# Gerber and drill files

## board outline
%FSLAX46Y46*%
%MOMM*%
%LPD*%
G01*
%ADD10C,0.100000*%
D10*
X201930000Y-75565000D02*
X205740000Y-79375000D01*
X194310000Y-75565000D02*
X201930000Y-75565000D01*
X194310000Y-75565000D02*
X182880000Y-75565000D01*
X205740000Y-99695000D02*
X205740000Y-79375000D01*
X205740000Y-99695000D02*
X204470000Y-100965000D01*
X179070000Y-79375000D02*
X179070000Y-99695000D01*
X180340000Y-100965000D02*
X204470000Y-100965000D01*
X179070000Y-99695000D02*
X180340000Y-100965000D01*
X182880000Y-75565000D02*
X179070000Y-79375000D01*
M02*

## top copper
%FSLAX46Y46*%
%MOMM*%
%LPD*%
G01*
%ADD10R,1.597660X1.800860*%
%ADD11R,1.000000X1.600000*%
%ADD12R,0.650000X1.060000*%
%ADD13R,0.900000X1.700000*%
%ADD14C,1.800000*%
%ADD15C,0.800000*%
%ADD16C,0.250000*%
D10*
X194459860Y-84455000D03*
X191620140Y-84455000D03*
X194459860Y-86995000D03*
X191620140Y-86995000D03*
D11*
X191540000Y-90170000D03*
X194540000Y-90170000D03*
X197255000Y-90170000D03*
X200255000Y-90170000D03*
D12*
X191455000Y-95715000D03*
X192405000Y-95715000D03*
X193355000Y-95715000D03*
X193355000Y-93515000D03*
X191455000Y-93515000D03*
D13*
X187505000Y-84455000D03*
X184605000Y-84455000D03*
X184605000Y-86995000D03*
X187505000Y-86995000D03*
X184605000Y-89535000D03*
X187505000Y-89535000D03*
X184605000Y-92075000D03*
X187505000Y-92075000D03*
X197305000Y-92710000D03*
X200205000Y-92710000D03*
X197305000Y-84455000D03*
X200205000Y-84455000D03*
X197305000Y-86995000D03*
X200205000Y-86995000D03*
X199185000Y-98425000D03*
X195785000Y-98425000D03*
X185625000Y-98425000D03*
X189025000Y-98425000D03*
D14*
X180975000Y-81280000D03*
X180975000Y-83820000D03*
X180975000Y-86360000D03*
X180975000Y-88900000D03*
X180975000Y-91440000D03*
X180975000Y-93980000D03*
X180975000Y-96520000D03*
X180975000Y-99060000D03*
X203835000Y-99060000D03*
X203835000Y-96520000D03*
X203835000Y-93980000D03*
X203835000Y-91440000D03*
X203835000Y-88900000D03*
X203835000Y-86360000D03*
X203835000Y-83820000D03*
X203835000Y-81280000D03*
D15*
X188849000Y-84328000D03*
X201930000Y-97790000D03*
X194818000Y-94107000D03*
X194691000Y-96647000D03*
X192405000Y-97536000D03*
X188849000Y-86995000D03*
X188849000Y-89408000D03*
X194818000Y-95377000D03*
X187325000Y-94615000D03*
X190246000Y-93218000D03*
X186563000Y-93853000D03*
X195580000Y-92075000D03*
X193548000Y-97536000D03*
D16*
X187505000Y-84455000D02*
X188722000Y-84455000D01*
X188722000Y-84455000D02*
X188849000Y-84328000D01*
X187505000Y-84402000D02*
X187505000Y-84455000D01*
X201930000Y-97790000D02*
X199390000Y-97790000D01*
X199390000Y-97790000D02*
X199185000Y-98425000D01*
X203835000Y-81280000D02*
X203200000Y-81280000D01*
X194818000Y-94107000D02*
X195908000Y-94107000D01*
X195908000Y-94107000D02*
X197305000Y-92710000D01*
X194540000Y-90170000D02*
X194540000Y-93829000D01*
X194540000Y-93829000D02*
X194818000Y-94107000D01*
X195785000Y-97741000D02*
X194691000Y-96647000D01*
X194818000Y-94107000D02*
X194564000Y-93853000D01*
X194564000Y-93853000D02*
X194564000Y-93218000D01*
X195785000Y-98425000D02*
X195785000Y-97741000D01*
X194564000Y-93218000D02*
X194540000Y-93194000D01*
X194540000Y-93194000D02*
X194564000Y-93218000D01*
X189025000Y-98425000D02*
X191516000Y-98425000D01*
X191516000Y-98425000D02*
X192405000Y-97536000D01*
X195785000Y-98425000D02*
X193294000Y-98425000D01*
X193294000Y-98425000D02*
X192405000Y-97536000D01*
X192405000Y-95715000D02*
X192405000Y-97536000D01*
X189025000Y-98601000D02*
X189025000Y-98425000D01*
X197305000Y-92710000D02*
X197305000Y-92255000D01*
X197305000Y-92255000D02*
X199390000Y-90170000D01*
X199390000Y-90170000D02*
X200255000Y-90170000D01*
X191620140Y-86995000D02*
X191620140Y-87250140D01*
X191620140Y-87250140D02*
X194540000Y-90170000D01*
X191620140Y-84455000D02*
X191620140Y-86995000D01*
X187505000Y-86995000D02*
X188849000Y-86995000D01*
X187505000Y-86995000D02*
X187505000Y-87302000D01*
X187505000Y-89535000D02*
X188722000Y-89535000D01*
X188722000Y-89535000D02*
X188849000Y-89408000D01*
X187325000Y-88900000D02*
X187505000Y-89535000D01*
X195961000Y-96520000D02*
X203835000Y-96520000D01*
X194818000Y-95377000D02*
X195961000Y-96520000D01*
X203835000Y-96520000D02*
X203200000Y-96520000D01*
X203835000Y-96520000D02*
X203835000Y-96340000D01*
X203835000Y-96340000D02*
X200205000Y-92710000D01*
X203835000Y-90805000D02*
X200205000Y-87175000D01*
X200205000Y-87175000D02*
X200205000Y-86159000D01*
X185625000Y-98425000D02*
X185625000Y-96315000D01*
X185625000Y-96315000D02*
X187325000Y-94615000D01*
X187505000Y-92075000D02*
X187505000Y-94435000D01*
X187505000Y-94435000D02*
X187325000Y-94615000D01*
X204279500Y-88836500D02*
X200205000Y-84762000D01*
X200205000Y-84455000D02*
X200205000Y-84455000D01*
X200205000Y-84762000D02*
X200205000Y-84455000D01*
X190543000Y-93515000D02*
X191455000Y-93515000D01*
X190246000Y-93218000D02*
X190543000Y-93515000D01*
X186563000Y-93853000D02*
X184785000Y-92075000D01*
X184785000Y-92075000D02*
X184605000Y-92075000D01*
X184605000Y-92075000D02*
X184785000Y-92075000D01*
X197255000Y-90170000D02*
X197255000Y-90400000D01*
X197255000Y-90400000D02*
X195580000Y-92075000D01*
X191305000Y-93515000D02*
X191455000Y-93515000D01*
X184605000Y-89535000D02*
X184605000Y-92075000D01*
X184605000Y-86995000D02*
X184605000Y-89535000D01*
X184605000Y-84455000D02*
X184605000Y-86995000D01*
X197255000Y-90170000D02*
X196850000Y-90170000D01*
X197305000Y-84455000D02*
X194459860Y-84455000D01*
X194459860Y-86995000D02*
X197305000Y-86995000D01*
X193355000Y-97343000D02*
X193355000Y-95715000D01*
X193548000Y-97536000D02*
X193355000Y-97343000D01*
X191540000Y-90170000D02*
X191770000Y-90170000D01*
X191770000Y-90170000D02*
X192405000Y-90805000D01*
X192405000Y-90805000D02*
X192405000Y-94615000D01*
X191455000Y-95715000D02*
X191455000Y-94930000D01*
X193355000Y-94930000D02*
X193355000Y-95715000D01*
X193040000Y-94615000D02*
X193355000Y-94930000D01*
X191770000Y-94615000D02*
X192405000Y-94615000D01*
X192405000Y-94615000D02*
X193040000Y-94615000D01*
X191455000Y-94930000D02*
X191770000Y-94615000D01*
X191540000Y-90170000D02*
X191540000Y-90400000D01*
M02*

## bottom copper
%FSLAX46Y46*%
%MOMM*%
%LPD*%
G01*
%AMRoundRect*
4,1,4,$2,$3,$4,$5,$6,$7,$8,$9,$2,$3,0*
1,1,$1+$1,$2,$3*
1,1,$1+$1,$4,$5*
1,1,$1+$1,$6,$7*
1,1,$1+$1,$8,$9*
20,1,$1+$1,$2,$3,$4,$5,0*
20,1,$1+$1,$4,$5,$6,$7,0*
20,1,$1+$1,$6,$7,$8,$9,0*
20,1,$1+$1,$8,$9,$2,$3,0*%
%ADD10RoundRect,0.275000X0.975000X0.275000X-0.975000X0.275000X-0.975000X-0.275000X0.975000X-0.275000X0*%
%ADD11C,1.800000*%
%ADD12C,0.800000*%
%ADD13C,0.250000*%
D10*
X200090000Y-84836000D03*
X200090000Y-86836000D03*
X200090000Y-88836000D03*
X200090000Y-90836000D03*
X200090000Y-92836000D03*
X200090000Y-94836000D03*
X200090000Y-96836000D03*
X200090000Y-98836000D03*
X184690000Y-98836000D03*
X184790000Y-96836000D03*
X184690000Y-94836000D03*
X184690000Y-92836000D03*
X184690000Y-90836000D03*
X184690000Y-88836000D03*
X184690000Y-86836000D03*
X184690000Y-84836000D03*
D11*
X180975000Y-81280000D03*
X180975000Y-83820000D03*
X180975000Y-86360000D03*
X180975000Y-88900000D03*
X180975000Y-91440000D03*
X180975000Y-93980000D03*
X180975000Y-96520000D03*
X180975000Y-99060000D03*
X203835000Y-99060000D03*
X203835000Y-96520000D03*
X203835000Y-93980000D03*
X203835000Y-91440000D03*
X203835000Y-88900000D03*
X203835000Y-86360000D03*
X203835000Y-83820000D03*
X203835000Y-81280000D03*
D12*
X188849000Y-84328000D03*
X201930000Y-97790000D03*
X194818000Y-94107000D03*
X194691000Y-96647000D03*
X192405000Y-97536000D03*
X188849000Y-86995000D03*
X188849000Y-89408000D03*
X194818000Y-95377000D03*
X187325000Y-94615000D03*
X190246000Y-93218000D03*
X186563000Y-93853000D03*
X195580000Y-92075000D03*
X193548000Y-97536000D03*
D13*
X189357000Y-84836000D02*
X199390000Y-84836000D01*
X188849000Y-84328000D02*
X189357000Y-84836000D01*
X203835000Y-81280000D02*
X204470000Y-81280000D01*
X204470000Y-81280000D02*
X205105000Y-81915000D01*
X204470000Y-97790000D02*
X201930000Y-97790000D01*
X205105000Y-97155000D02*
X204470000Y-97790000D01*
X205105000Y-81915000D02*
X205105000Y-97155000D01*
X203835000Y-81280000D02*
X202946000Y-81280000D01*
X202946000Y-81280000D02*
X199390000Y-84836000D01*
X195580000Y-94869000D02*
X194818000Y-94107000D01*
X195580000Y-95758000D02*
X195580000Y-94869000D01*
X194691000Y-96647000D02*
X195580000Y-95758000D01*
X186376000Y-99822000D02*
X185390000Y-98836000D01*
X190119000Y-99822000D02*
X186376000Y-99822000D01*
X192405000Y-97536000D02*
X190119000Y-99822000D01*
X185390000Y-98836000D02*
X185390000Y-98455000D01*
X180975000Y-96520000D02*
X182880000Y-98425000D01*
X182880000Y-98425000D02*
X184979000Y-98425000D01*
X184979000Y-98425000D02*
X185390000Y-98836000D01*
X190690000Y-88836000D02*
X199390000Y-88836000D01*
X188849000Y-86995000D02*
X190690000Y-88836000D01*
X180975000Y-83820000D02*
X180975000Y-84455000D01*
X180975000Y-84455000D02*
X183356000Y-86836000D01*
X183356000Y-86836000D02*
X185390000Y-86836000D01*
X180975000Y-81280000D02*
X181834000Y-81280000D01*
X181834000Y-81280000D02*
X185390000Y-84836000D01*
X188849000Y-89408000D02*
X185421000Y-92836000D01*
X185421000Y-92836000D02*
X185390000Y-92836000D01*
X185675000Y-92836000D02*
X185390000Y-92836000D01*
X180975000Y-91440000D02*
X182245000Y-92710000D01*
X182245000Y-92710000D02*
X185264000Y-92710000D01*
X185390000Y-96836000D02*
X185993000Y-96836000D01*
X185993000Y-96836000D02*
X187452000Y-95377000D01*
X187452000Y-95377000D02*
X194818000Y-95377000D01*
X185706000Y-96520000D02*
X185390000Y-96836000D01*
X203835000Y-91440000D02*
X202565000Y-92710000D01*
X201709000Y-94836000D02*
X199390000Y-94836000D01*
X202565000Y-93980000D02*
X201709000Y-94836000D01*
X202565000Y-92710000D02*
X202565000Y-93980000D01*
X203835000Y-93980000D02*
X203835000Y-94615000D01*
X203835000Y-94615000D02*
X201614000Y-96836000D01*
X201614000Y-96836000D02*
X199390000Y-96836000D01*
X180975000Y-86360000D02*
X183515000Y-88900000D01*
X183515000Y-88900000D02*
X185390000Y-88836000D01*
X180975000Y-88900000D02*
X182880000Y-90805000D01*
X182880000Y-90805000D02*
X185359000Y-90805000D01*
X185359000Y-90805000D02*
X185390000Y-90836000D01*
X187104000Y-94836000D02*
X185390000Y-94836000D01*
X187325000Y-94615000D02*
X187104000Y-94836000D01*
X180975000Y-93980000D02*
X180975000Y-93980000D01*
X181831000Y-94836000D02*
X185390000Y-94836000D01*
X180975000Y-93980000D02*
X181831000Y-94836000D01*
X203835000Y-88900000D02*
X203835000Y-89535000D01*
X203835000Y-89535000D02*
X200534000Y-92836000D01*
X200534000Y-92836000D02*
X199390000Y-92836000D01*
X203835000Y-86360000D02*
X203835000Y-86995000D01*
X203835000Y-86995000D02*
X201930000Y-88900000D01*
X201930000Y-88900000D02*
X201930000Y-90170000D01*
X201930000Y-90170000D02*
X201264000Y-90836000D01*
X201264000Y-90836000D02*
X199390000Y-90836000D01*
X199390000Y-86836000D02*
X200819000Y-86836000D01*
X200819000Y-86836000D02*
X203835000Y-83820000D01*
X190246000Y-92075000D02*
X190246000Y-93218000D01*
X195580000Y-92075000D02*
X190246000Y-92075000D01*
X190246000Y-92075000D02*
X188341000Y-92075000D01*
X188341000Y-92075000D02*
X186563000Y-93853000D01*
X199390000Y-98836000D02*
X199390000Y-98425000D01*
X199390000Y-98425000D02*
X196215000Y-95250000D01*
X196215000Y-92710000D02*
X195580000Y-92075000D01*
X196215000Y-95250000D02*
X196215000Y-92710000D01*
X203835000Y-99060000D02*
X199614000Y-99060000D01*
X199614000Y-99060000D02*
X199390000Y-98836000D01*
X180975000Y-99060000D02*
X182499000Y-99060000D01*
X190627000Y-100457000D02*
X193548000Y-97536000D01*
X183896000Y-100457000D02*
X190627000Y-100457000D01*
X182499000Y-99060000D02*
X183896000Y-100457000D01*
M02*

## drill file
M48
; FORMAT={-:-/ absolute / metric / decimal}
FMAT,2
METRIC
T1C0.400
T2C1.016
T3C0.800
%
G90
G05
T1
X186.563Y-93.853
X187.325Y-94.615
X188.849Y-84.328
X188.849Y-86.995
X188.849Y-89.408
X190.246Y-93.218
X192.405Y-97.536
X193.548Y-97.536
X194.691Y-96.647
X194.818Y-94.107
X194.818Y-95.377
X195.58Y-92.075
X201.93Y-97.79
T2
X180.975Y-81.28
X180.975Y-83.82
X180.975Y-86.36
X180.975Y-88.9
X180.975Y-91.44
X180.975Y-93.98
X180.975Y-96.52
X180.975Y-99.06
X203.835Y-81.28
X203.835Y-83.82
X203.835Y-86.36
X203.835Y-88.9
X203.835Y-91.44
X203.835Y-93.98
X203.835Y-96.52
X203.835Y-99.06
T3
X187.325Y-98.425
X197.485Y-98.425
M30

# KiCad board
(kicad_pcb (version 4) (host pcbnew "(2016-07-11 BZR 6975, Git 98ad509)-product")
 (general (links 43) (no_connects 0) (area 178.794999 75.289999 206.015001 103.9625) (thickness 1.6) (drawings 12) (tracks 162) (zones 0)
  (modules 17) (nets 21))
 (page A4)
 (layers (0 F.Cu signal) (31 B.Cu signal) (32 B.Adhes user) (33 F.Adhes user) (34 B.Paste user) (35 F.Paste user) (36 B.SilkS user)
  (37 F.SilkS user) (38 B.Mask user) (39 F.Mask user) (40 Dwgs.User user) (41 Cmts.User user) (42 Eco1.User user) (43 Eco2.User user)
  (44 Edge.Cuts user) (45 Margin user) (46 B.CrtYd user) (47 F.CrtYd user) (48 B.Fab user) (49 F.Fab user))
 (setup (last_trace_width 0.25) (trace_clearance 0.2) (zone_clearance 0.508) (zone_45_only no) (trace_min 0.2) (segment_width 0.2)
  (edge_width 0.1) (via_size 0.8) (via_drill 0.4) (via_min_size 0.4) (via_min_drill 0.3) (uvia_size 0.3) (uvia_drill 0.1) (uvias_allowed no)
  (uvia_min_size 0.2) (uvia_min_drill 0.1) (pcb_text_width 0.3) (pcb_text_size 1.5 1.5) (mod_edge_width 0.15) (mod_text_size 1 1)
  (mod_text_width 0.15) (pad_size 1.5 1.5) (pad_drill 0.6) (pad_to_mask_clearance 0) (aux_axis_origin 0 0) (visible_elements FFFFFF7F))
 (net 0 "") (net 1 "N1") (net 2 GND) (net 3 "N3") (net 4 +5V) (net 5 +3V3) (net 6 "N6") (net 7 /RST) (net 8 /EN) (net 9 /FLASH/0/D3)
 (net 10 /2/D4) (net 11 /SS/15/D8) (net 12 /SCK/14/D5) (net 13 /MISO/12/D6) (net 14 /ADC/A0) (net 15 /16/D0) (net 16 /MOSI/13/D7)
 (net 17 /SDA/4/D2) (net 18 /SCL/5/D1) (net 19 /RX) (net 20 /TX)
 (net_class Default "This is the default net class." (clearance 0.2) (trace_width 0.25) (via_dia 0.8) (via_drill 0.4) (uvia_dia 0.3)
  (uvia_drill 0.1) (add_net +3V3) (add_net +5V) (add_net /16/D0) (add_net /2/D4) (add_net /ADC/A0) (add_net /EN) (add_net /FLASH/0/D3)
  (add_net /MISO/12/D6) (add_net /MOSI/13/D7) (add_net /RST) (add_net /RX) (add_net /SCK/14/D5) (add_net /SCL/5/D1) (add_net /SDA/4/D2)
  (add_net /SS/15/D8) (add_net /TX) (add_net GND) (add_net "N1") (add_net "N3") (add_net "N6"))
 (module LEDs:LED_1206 (layer F.Cu) (at 193.04 84.455)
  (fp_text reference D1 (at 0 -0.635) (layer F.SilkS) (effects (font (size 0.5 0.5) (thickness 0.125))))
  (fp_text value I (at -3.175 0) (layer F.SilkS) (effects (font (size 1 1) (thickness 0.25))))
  (pad 2 smd rect (at 1.41986 0 180) (size 1.59766 1.80086) (layers F.Cu F.Paste F.Mask) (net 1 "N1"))
  (pad 1 smd rect (at -1.41986 0 180) (size 1.59766 1.80086) (layers F.Cu F.Paste F.Mask) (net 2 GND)))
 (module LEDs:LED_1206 (layer F.Cu) (at 193.04 86.995)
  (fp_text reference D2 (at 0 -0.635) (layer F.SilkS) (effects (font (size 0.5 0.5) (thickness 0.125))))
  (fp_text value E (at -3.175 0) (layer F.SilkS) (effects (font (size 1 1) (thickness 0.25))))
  (pad 2 smd rect (at 1.41986 0 180) (size 1.59766 1.80086) (layers F.Cu F.Paste F.Mask) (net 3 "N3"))
  (pad 1 smd rect (at -1.41986 0 180) (size 1.59766 1.80086) (layers F.Cu F.Paste F.Mask) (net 2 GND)))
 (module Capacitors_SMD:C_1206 (layer F.Cu) (at 193.04 90.17)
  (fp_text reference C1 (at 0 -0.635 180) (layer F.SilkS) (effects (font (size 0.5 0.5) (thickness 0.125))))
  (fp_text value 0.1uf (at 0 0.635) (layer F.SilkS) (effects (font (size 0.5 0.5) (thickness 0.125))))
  (pad 1 smd rect (at -1.5 0) (size 1 1.6) (layers F.Cu F.Paste F.Mask) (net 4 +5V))
  (pad 2 smd rect (at 1.5 0) (size 1 1.6) (layers F.Cu F.Paste F.Mask) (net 2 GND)))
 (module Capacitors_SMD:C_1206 (layer F.Cu) (at 198.755 90.17)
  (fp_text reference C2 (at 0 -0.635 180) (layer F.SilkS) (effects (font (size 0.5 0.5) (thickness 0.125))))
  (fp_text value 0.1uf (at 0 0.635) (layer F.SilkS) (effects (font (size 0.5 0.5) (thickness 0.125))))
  (pad 1 smd rect (at -1.5 0) (size 1 1.6) (layers F.Cu F.Paste F.Mask) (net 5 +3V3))
  (pad 2 smd rect (at 1.5 0) (size 1 1.6) (layers F.Cu F.Paste F.Mask) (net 2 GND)))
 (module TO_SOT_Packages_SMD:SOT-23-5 (layer F.Cu) (at 192.405 94.615 90)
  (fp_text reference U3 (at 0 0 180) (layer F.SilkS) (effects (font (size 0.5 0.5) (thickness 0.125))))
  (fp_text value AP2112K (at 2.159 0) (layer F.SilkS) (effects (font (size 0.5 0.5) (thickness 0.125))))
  (pad 1 smd rect (at -1.1 -0.95 90) (size 1.06 0.65) (layers F.Cu F.Paste F.Mask) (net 4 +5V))
  (pad 2 smd rect (at -1.1 0 90) (size 1.06 0.65) (layers F.Cu F.Paste F.Mask) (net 2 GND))
  (pad 3 smd rect (at -1.1 0.95 90) (size 1.06 0.65) (layers F.Cu F.Paste F.Mask) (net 4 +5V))
  (pad 4 smd rect (at 1.1 0.95 90) (size 1.06 0.65) (layers F.Cu F.Paste F.Mask) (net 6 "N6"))
  (pad 5 smd rect (at 1.1 -0.95 90) (size 1.06 0.65) (layers F.Cu F.Paste F.Mask) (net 5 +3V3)))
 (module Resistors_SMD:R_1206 (layer F.Cu) (at 186.055 84.455 180)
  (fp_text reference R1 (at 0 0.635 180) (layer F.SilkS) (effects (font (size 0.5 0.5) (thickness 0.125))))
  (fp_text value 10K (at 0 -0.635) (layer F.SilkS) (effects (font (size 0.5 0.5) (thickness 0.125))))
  (pad 1 smd rect (at -1.45 0 180) (size 0.9 1.7) (layers F.Cu F.Paste F.Mask) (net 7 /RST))
  (pad 2 smd rect (at 1.45 0 180) (size 0.9 1.7) (layers F.Cu F.Paste F.Mask) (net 5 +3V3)))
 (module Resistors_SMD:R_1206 (layer F.Cu) (at 186.055 86.995)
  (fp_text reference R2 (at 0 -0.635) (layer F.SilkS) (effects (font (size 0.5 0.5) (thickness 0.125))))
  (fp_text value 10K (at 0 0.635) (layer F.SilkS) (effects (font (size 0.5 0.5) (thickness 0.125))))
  (pad 1 smd rect (at -1.45 0) (size 0.9 1.7) (layers F.Cu F.Paste F.Mask) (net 5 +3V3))
  (pad 2 smd rect (at 1.45 0) (size 0.9 1.7) (layers F.Cu F.Paste F.Mask) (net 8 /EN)))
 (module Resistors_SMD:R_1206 (layer F.Cu) (at 186.055 89.535)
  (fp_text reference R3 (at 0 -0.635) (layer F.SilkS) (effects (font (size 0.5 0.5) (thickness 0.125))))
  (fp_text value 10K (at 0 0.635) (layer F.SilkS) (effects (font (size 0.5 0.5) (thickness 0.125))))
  (pad 1 smd rect (at -1.45 0) (size 0.9 1.7) (layers F.Cu F.Paste F.Mask) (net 5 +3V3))
  (pad 2 smd rect (at 1.45 0) (size 0.9 1.7) (layers F.Cu F.Paste F.Mask) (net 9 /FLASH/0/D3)))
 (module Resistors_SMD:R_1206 (layer F.Cu) (at 186.055 92.075)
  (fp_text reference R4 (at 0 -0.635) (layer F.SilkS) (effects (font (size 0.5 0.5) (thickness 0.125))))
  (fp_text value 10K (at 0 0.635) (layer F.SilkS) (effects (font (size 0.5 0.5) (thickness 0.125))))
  (pad 1 smd rect (at -1.45 0) (size 0.9 1.7) (layers F.Cu F.Paste F.Mask) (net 5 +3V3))
  (pad 2 smd rect (at 1.45 0) (size 0.9 1.7) (layers F.Cu F.Paste F.Mask) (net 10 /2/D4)))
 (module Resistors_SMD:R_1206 (layer F.Cu) (at 198.755 92.71)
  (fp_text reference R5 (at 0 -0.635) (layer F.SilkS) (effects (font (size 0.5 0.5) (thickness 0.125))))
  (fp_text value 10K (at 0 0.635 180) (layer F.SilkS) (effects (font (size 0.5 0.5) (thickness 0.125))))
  (pad 1 smd rect (at -1.45 0) (size 0.9 1.7) (layers F.Cu F.Paste F.Mask) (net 2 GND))
  (pad 2 smd rect (at 1.45 0) (size 0.9 1.7) (layers F.Cu F.Paste F.Mask) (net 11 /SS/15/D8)))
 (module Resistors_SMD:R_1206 (layer F.Cu) (at 198.755 84.455)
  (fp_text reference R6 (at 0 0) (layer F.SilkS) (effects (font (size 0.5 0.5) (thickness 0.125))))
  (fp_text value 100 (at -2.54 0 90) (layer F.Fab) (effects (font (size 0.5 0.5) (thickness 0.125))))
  (pad 1 smd rect (at -1.45 0) (size 0.9 1.7) (layers F.Cu F.Paste F.Mask) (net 1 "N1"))
  (pad 2 smd rect (at 1.45 0) (size 0.9 1.7) (layers F.Cu F.Paste F.Mask) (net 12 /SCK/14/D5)))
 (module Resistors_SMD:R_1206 (layer F.Cu) (at 198.755 86.995)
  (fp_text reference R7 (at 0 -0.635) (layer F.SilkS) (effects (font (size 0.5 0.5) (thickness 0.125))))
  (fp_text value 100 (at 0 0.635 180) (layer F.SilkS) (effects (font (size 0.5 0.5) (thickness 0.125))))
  (pad 1 smd rect (at -1.45 0) (size 0.9 1.7) (layers F.Cu F.Paste F.Mask) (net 3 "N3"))
  (pad 2 smd rect (at 1.45 0) (size 0.9 1.7) (layers F.Cu F.Paste F.Mask) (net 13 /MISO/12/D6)))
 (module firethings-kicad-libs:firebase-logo (layer F.Cu) (at 197.993 79.248)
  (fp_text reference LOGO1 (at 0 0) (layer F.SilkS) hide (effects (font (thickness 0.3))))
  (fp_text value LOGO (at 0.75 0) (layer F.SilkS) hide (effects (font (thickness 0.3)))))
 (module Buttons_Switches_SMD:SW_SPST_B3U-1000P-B (layer F.Cu) (at 197.485 98.425 180)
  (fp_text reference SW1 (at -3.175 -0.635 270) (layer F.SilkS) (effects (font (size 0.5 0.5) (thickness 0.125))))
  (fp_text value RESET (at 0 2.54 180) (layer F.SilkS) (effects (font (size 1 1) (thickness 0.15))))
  (pad 1 smd rect (at -1.7 0 180) (size 0.9 1.7) (layers F.Cu F.Paste F.Mask) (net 7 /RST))
  (pad 2 smd rect (at 1.7 0 180) (size 0.9 1.7) (layers F.Cu F.Paste F.Mask) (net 2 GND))
  (pad "" np_thru_hole circle (at 0 0 180) (size 0.8 0.8) (drill 0.8) (layers *.Cu *.Mask)))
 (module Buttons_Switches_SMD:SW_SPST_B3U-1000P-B (layer F.Cu) (at 187.325 98.425)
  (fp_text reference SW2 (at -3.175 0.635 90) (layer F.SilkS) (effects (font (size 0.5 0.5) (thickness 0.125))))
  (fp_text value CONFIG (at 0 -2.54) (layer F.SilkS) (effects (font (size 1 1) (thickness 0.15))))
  (pad 1 smd rect (at -1.7 0) (size 0.9 1.7) (layers F.Cu F.Paste F.Mask) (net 10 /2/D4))
  (pad 2 smd rect (at 1.7 0) (size 0.9 1.7) (layers F.Cu F.Paste F.Mask) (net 2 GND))
  (pad "" np_thru_hole circle (at 0 0) (size 0.8 0.8) (drill 0.8) (layers *.Cu *.Mask)))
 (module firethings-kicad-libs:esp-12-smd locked (layer B.Cu) (at 199.39 84.836 180)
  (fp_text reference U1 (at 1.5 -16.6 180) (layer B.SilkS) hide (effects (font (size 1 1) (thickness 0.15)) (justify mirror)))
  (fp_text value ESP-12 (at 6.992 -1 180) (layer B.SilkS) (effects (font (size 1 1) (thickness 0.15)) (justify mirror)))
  (pad 1 smd roundrect (at 0 0 180) (size 2.5 1.1) (drill (offset -0.7 0)) (layers B.Cu B.Paste B.Mask) (roundrect_rratio 0.25) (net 7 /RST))
  (pad 2 smd roundrect (at 0 -2 180) (size 2.5 1.1) (drill (offset -0.7 0)) (layers B.Cu B.Paste B.Mask) (roundrect_rratio 0.25)
   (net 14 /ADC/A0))
  (pad 3 smd roundrect (at 0 -4 180) (size 2.5 1.1) (drill (offset -0.7 0)) (layers B.Cu B.Paste B.Mask) (roundrect_rratio 0.25) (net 8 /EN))
  (pad 4 smd roundrect (at 0 -6 180) (size 2.5 1.1) (drill (offset -0.7 0)) (layers B.Cu B.Paste B.Mask) (roundrect_rratio 0.25)
   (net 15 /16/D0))
  (pad 5 smd roundrect (at 0 -8 180) (size 2.5 1.1) (drill (offset -0.7 0)) (layers B.Cu B.Paste B.Mask) (roundrect_rratio 0.25)
   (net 12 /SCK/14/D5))
  (pad 6 smd roundrect (at 0 -10 180) (size 2.5 1.1) (drill (offset -0.7 0)) (layers B.Cu B.Paste B.Mask) (roundrect_rratio 0.25)
   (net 13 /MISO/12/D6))
  (pad 7 smd roundrect (at 0 -12 180) (size 2.5 1.1) (drill (offset -0.7 0)) (layers B.Cu B.Paste B.Mask) (roundrect_rratio 0.25)
   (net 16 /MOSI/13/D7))
  (pad 8 smd roundrect (at 0 -14 180) (size 2.5 1.1) (drill (offset -0.7 0)) (layers B.Cu B.Paste B.Mask) (roundrect_rratio 0.25)
   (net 5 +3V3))
  (pad 9 smd roundrect (at 14 -14 180) (size 2.5 1.1) (drill (offset 0.7 0)) (layers B.Cu B.Paste B.Mask) (roundrect_rratio 0.25)
   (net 2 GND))
  (pad 10 smd roundrect (at 14 -12 180) (size 2.5 1.1) (drill (offset 0.6 0)) (layers B.Cu B.Paste B.Mask) (roundrect_rratio 0.25)
   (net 11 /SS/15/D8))
  (pad 11 smd roundrect (at 14 -10 180) (size 2.5 1.1) (drill (offset 0.7 0)) (layers B.Cu B.Paste B.Mask) (roundrect_rratio 0.25)
   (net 10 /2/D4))
  (pad 12 smd roundrect (at 14 -8 180) (size 2.5 1.1) (drill (offset 0.7 0)) (layers B.Cu B.Paste B.Mask) (roundrect_rratio 0.25)
   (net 9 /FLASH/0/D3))
  (pad 13 smd roundrect (at 14 -6 180) (size 2.5 1.1) (drill (offset 0.7 0)) (layers B.Cu B.Paste B.Mask) (roundrect_rratio 0.25)
   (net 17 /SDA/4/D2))
  (pad 14 smd roundrect (at 14 -4 180) (size 2.5 1.1) (drill (offset 0.7 0)) (layers B.Cu B.Paste B.Mask) (roundrect_rratio 0.25)
   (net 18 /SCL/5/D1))
  (pad 15 smd roundrect (at 14 -2 180) (size 2.5 1.1) (drill (offset 0.7 0)) (layers B.Cu B.Paste B.Mask) (roundrect_rratio 0.25)
   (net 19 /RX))
  (pad 16 smd roundrect (at 14 0 180) (size 2.5 1.1) (drill (offset 0.7 0)) (layers B.Cu B.Paste B.Mask) (roundrect_rratio 0.25)
   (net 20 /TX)))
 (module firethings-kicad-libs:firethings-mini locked (layer F.Cu) (at 192.405 91.44)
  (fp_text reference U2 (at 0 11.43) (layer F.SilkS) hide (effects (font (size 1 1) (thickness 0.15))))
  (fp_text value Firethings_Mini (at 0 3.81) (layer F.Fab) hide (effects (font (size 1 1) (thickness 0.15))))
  (pad 8 thru_hole circle (at -11.43 -10.16) (size 1.8 1.8) (drill 1.016) (layers *.Cu *.Mask F.SilkS) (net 20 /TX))
  (pad 7 thru_hole circle (at -11.43 -7.62) (size 1.8 1.8) (drill 1.016) (layers *.Cu *.Mask F.SilkS) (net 19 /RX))
  (pad 6 thru_hole circle (at -11.43 -5.08) (size 1.8 1.8) (drill 1.016) (layers *.Cu *.Mask F.SilkS) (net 18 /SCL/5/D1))
  (pad 5 thru_hole circle (at -11.43 -2.54) (size 1.8 1.8) (drill 1.016) (layers *.Cu *.Mask F.SilkS) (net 17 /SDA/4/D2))
  (pad 4 thru_hole circle (at -11.43 0) (size 1.8 1.8) (drill 1.016) (layers *.Cu *.Mask F.SilkS) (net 9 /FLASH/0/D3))
  (pad 3 thru_hole circle (at -11.43 2.54) (size 1.8 1.8) (drill 1.016) (layers *.Cu *.Mask F.SilkS) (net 10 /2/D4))
  (pad 2 thru_hole circle (at -11.43 5.08) (size 1.8 1.8) (drill 1.016) (layers *.Cu *.Mask F.SilkS) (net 2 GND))
  (pad 1 thru_hole circle (at -11.43 7.62) (size 1.8 1.8) (drill 1.016) (layers *.Cu *.Mask F.SilkS) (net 4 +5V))
  (pad 16 thru_hole circle (at 11.43 7.62) (size 1.8 1.8) (drill 1.016) (layers *.Cu *.Mask F.SilkS) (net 5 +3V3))
  (pad 15 thru_hole circle (at 11.43 5.08) (size 1.8 1.8) (drill 1.016) (layers *.Cu *.Mask F.SilkS) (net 11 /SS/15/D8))
  (pad 14 thru_hole circle (at 11.43 2.54) (size 1.8 1.8) (drill 1.016) (layers *.Cu *.Mask F.SilkS) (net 16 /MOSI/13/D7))
  (pad 13 thru_hole circle (at 11.43 0) (size 1.8 1.8) (drill 1.016) (layers *.Cu *.Mask F.SilkS) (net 13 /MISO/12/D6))
  (pad 12 thru_hole circle (at 11.43 -2.54) (size 1.8 1.8) (drill 1.016) (layers *.Cu *.Mask F.SilkS) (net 12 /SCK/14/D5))
  (pad 11 thru_hole circle (at 11.43 -5.08) (size 1.8 1.8) (drill 1.016) (layers *.Cu *.Mask F.SilkS) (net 15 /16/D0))
  (pad 10 thru_hole circle (at 11.43 -7.62) (size 1.8 1.8) (drill 1.016) (layers *.Cu *.Mask F.SilkS) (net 14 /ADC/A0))
  (pad 9 thru_hole circle (at 11.43 -10.16) (size 1.8 1.8) (drill 1.016) (layers *.Cu *.Mask F.SilkS) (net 7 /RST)))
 (gr_line (start 201.93 75.565) (end 205.74 79.375) (angle 90) (layer Edge.Cuts) (width 0.1))
 (gr_line (start 194.31 75.565) (end 201.93 75.565) (angle 90) (layer Edge.Cuts) (width 0.1))
 (gr_line (start 194.31 75.565) (end 182.88 75.565) (angle 90) (layer Edge.Cuts) (width 0.1))
 (gr_line (start 205.74 99.695) (end 205.74 79.375) (angle 90) (layer Edge.Cuts) (width 0.1))
 (gr_line (start 205.74 99.695) (end 204.47 100.965) (angle 90) (layer Edge.Cuts) (width 0.1))
 (gr_line (start 179.07 79.375) (end 179.07 99.695) (angle 90) (layer Edge.Cuts) (width 0.1))
 (gr_line (start 180.34 100.965) (end 204.47 100.965) (angle 90) (layer Edge.Cuts) (width 0.1))
 (gr_line (start 179.07 99.695) (end 180.34 100.965) (angle 90) (layer Edge.Cuts) (width 0.1))
 (gr_line (start 182.88 75.565) (end 179.07 79.375) (angle 90) (layer Edge.Cuts) (width 0.1))
 (segment (start 187.505 84.455) (end 188.722 84.455) (width 0.25) (layer F.Cu) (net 7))
 (segment (start 189.357 84.836) (end 199.39 84.836) (width 0.25) (layer B.Cu) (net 7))
 (segment (start 188.849 84.328) (end 189.357 84.836) (width 0.25) (layer B.Cu) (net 7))
 (via (at 188.849 84.328) (size 0.8) (drill 0.4) (layers F.Cu B.Cu) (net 7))
 (segment (start 188.722 84.455) (end 188.849 84.328) (width 0.25) (layer F.Cu) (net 7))
 (segment (start 187.505 84.402) (end 187.505 84.455) (width 0.25) (layer F.Cu) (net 7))
 (segment (start 203.835 81.28) (end 204.47 81.28) (width 0.25) (layer B.Cu) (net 7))
 (segment (start 204.47 81.28) (end 205.105 81.915) (width 0.25) (layer B.Cu) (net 7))
 (segment (start 201.93 97.79) (end 199.39 97.79) (width 0.25) (layer F.Cu) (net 7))
 (via (at 201.93 97.79) (size 0.8) (drill 0.4) (layers F.Cu B.Cu) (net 7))
 (segment (start 204.47 97.79) (end 201.93 97.79) (width 0.25) (layer B.Cu) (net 7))
 (segment (start 205.105 97.155) (end 204.47 97.79) (width 0.25) (layer B.Cu) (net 7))
 (segment (start 205.105 81.915) (end 205.105 97.155) (width 0.25) (layer B.Cu) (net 7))
 (segment (start 199.39 97.79) (end 199.185 98.425) (width 0.25) (layer F.Cu) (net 7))
 (segment (start 203.835 81.28) (end 202.946 81.28) (width 0.25) (layer B.Cu) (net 7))
 (segment (start 202.946 81.28) (end 199.39 84.836) (width 0.25) (layer B.Cu) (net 7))
 (segment (start 203.835 81.28) (end 203.2 81.28) (width 0.25) (layer F.Cu) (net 7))
 (segment (start 194.818 94.107) (end 195.908 94.107) (width 0.25) (layer F.Cu) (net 2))
 (segment (start 195.908 94.107) (end 197.305 92.71) (width 0.25) (layer F.Cu) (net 2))
 (segment (start 194.54 90.17) (end 194.54 93.829) (width 0.25) (layer F.Cu) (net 2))
 (segment (start 194.54 93.829) (end 194.818 94.107) (width 0.25) (layer F.Cu) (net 2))
 (segment (start 195.785 97.741) (end 194.691 96.647) (width 0.25) (layer F.Cu) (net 2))
 (via (at 194.818 94.107) (size 0.8) (drill 0.4) (layers F.Cu B.Cu) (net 2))
 (segment (start 195.58 94.869) (end 194.818 94.107) (width 0.25) (layer B.Cu) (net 2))
 (segment (start 195.58 95.758) (end 195.58 94.869) (width 0.25) (layer B.Cu) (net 2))
 (segment (start 194.691 96.647) (end 195.58 95.758) (width 0.25) (layer B.Cu) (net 2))
 (via (at 194.691 96.647) (size 0.8) (drill 0.4) (layers F.Cu B.Cu) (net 2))
 (segment (start 194.818 94.107) (end 194.564 93.853) (width 0.25) (layer F.Cu) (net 2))
 (segment (start 194.564 93.853) (end 194.564 93.218) (width 0.25) (layer F.Cu) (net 2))
 (segment (start 195.785 98.425) (end 195.785 97.741) (width 0.25) (layer F.Cu) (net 2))
 (segment (start 194.564 93.218) (end 194.54 93.194) (width 0.25) (layer F.Cu) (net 2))
 (segment (start 194.54 93.194) (end 194.564 93.218) (width 0.25) (layer F.Cu) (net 2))
 (segment (start 189.025 98.425) (end 191.516 98.425) (width 0.25) (layer F.Cu) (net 2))
 (segment (start 191.516 98.425) (end 192.405 97.536) (width 0.25) (layer F.Cu) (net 2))
 (segment (start 195.785 98.425) (end 193.294 98.425) (width 0.25) (layer F.Cu) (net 2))
 (segment (start 193.294 98.425) (end 192.405 97.536) (width 0.25) (layer F.Cu) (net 2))
 (segment (start 192.405 95.715) (end 192.405 97.536) (width 0.25) (layer F.Cu) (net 2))
 (segment (start 186.376 99.822) (end 185.39 98.836) (width 0.25) (layer B.Cu) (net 2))
 (segment (start 190.119 99.822) (end 186.376 99.822) (width 0.25) (layer B.Cu) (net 2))
 (segment (start 192.405 97.536) (end 190.119 99.822) (width 0.25) (layer B.Cu) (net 2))
 (via (at 192.405 97.536) (size 0.8) (drill 0.4) (layers F.Cu B.Cu) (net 2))
 (segment (start 189.025 98.601) (end 189.025 98.425) (width 0.25) (layer F.Cu) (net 2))
 (segment (start 185.39 98.836) (end 185.39 98.455) (width 0.25) (layer B.Cu) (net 2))
 (segment (start 197.305 92.71) (end 197.305 92.255) (width 0.25) (layer F.Cu) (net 2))
 (segment (start 197.305 92.255) (end 199.39 90.17) (width 0.25) (layer F.Cu) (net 2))
 (segment (start 199.39 90.17) (end 200.255 90.17) (width 0.25) (layer F.Cu) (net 2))
 (segment (start 191.62014 86.995) (end 191.62014 87.25014) (width 0.25) (layer F.Cu) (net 2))
 (segment (start 191.62014 87.25014) (end 194.54 90.17) (width 0.25) (layer F.Cu) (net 2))
 (segment (start 180.975 96.52) (end 182.88 98.425) (width 0.25) (layer B.Cu) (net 2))
 (segment (start 182.88 98.425) (end 184.979 98.425) (width 0.25) (layer B.Cu) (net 2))
 (segment (start 184.979 98.425) (end 185.39 98.836) (width 0.25) (layer B.Cu) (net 2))
 (segment (start 191.62014 84.455) (end 191.62014 86.995) (width 0.25) (layer F.Cu) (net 2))
 (segment (start 187.505 86.995) (end 188.849 86.995) (width 0.25) (layer F.Cu) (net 8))
 (segment (start 190.69 88.836) (end 199.39 88.836) (width 0.25) (layer B.Cu) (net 8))
 (segment (start 188.849 86.995) (end 190.69 88.836) (width 0.25) (layer B.Cu) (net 8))
 (via (at 188.849 86.995) (size 0.8) (drill 0.4) (layers F.Cu B.Cu) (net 8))
 (segment (start 187.505 86.995) (end 187.505 87.302) (width 0.25) (layer F.Cu) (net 8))
 (segment (start 180.975 83.82) (end 180.975 84.455) (width 0.25) (layer B.Cu) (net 19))
 (segment (start 180.975 84.455) (end 183.356 86.836) (width 0.25) (layer B.Cu) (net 19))
 (segment (start 183.356 86.836) (end 185.39 86.836) (width 0.25) (layer B.Cu) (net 19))
 (segment (start 180.975 81.28) (end 181.834 81.28) (width 0.25) (layer B.Cu) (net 20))
 (segment (start 181.834 81.28) (end 185.39 84.836) (width 0.25) (layer B.Cu) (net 20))
 (segment (start 187.505 89.535) (end 188.722 89.535) (width 0.25) (layer F.Cu) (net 9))
 (segment (start 188.849 89.408) (end 185.421 92.836) (width 0.25) (layer B.Cu) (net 9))
 (via (at 188.849 89.408) (size 0.8) (drill 0.4) (layers F.Cu B.Cu) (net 9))
 (segment (start 188.722 89.535) (end 188.849 89.408) (width 0.25) (layer F.Cu) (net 9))
 (segment (start 185.421 92.836) (end 185.39 92.836) (width 0.25) (layer B.Cu) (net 9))
 (segment (start 185.675 92.836) (end 185.39 92.836) (width 0.25) (layer B.Cu) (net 9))
 (segment (start 187.325 88.9) (end 187.505 89.535) (width 0.25) (layer F.Cu) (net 9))
 (segment (start 180.975 91.44) (end 182.245 92.71) (width 0.25) (layer B.Cu) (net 9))
 (segment (start 182.245 92.71) (end 185.264 92.71) (width 0.25) (layer B.Cu) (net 9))
 (segment (start 185.39 96.836) (end 185.993 96.836) (width 0.25) (layer B.Cu) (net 11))
 (segment (start 185.993 96.836) (end 187.452 95.377) (width 0.25) (layer B.Cu) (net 11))
 (segment (start 195.961 96.52) (end 203.835 96.52) (width 0.25) (layer F.Cu) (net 11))
 (segment (start 194.818 95.377) (end 195.961 96.52) (width 0.25) (layer F.Cu) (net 11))
 (via (at 194.818 95.377) (size 0.8) (drill 0.4) (layers F.Cu B.Cu) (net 11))
 (segment (start 187.452 95.377) (end 194.818 95.377) (width 0.25) (layer B.Cu) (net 11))
 (segment (start 203.835 96.52) (end 203.2 96.52) (width 0.25) (layer F.Cu) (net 11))
 (segment (start 185.706 96.52) (end 185.39 96.836) (width 0.25) (layer B.Cu) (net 11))
 (segment (start 203.835 96.52) (end 203.835 96.34) (width 0.25) (layer F.Cu) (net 11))
 (segment (start 203.835 96.34) (end 200.205 92.71) (width 0.25) (layer F.Cu) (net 11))
 (segment (start 203.835 90.805) (end 200.205 87.175) (width 0.25) (layer F.Cu) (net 13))
 (segment (start 200.205 87.175) (end 200.205 86.159) (width 0.25) (layer F.Cu) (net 13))
 (segment (start 203.835 91.44) (end 202.565 92.71) (width 0.25) (layer B.Cu) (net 13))
 (segment (start 201.709 94.836) (end 199.39 94.836) (width 0.25) (layer B.Cu) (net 13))
 (segment (start 202.565 93.98) (end 201.709 94.836) (width 0.25) (layer B.Cu) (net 13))
 (segment (start 202.565 92.71) (end 202.565 93.98) (width 0.25) (layer B.Cu) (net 13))
 (segment (start 203.835 93.98) (end 203.835 94.615) (width 0.25) (layer B.Cu) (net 16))
 (segment (start 203.835 94.615) (end 201.614 96.836) (width 0.25) (layer B.Cu) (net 16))
 (segment (start 201.614 96.836) (end 199.39 96.836) (width 0.25) (layer B.Cu) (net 16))
 (segment (start 180.975 86.36) (end 183.515 88.9) (width 0.25) (layer B.Cu) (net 18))
 (segment (start 183.515 88.9) (end 185.39 88.836) (width 0.25) (layer B.Cu) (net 18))
 (segment (start 180.975 88.9) (end 182.88 90.805) (width 0.25) (layer B.Cu) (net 17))
 (segment (start 182.88 90.805) (end 185.359 90.805) (width 0.25) (layer B.Cu) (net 17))
 (segment (start 185.359 90.805) (end 185.39 90.836) (width 0.25) (layer B.Cu) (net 17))
 (segment (start 185.625 98.425) (end 185.625 96.315) (width 0.25) (layer F.Cu) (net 10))
 (segment (start 185.625 96.315) (end 187.325 94.615) (width 0.25) (layer F.Cu) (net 10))
 (segment (start 187.505 92.075) (end 187.505 94.435) (width 0.25) (layer F.Cu) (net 10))
 (segment (start 187.104 94.836) (end 185.39 94.836) (width 0.25) (layer B.Cu) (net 10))
 (segment (start 187.325 94.615) (end 187.104 94.836) (width 0.25) (layer B.Cu) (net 10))
 (via (at 187.325 94.615) (size 0.8) (drill 0.4) (layers F.Cu B.Cu) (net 10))
 (segment (start 187.505 94.435) (end 187.325 94.615) (width 0.25) (layer F.Cu) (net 10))
 (segment (start 180.975 93.98) (end 180.975 93.98) (width 0.25) (layer B.Cu) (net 10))
 (segment (start 181.831 94.836) (end 185.39 94.836) (width 0.25) (layer B.Cu) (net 10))
 (segment (start 180.975 93.98) (end 181.831 94.836) (width 0.25) (layer B.Cu) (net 10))
 (segment (start 204.2795 88.8365) (end 200.205 84.762) (width 0.25) (layer F.Cu) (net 12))
 (segment (start 200.205 84.455) (end 200.205 84.455) (width 0.25) (layer F.Cu) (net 12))
 (segment (start 200.205 84.762) (end 200.205 84.455) (width 0.25) (layer F.Cu) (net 12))
 (segment (start 203.835 88.9) (end 203.835 89.535) (width 0.25) (layer B.Cu) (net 12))
 (segment (start 203.835 89.535) (end 200.534 92.836) (width 0.25) (layer B.Cu) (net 12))
 (segment (start 200.534 92.836) (end 199.39 92.836) (width 0.25) (layer B.Cu) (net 12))
 (segment (start 203.835 86.36) (end 203.835 86.995) (width 0.25) (layer B.Cu) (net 15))
 (segment (start 203.835 86.995) (end 201.93 88.9) (width 0.25) (layer B.Cu) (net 15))
 (segment (start 201.93 88.9) (end 201.93 90.17) (width 0.25) (layer B.Cu) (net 15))
 (segment (start 201.93 90.17) (end 201.264 90.836) (width 0.25) (layer B.Cu) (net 15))
 (segment (start 201.264 90.836) (end 199.39 90.836) (width 0.25) (layer B.Cu) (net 15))
 (segment (start 199.39 86.836) (end 200.819 86.836) (width 0.25) (layer B.Cu) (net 14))
 (segment (start 200.819 86.836) (end 203.835 83.82) (width 0.25) (layer B.Cu) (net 14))
 (segment (start 190.246 92.075) (end 190.246 93.218) (width 0.25) (layer B.Cu) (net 5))
 (segment (start 190.543 93.515) (end 191.455 93.515) (width 0.25) (layer F.Cu) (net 5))
 (segment (start 190.246 93.218) (end 190.543 93.515) (width 0.25) (layer F.Cu) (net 5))
 (via (at 190.246 93.218) (size 0.8) (drill 0.4) (layers F.Cu B.Cu) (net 5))
 (segment (start 195.58 92.075) (end 190.246 92.075) (width 0.25) (layer B.Cu) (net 5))
 (segment (start 190.246 92.075) (end 188.341 92.075) (width 0.25) (layer B.Cu) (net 5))
 (segment (start 186.563 93.853) (end 184.785 92.075) (width 0.25) (layer F.Cu) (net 5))
 (via (at 186.563 93.853) (size 0.8) (drill 0.4) (layers F.Cu B.Cu) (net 5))
 (segment (start 188.341 92.075) (end 186.563 93.853) (width 0.25) (layer B.Cu) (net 5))
 (segment (start 184.785 92.075) (end 184.605 92.075) (width 0.25) (layer F.Cu) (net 5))
 (segment (start 199.39 98.836) (end 199.39 98.425) (width 0.25) (layer B.Cu) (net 5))
 (segment (start 199.39 98.425) (end 196.215 95.25) (width 0.25) (layer B.Cu) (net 5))
 (segment (start 196.215 92.71) (end 195.58 92.075) (width 0.25) (layer B.Cu) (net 5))
 (segment (start 196.215 95.25) (end 196.215 92.71) (width 0.25) (layer B.Cu) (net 5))
 (segment (start 203.835 99.06) (end 199.614 99.06) (width 0.25) (layer B.Cu) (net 5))
 (segment (start 199.614 99.06) (end 199.39 98.836) (width 0.25) (layer B.Cu) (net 5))
 (segment (start 184.605 92.075) (end 184.785 92.075) (width 0.25) (layer F.Cu) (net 5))
 (segment (start 197.255 90.17) (end 197.255 90.4) (width 0.25) (layer F.Cu) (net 5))
 (segment (start 197.255 90.4) (end 195.58 92.075) (width 0.25) (layer F.Cu) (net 5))
 (via (at 195.58 92.075) (size 0.8) (drill 0.4) (layers F.Cu B.Cu) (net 5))
 (segment (start 191.305 93.515) (end 191.455 93.515) (width 0.25) (layer F.Cu) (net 5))
 (segment (start 184.605 89.535) (end 184.605 92.075) (width 0.25) (layer F.Cu) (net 5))
 (segment (start 184.605 86.995) (end 184.605 89.535) (width 0.25) (layer F.Cu) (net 5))
 (segment (start 184.605 84.455) (end 184.605 86.995) (width 0.25) (layer F.Cu) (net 5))
 (segment (start 197.255 90.17) (end 196.85 90.17) (width 0.25) (layer F.Cu) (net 5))
 (segment (start 197.305 84.455) (end 194.45986 84.455) (width 0.25) (layer F.Cu) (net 1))
 (segment (start 194.45986 86.995) (end 197.305 86.995) (width 0.25) (layer F.Cu) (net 3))
 (segment (start 180.975 99.06) (end 182.499 99.06) (width 0.25) (layer B.Cu) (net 4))
 (segment (start 193.355 97.343) (end 193.355 95.715) (width 0.25) (layer F.Cu) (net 4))
 (segment (start 193.548 97.536) (end 193.355 97.343) (width 0.25) (layer F.Cu) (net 4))
 (via (at 193.548 97.536) (size 0.8) (drill 0.4) (layers F.Cu B.Cu) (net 4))
 (segment (start 190.627 100.457) (end 193.548 97.536) (width 0.25) (layer B.Cu) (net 4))
 (segment (start 183.896 100.457) (end 190.627 100.457) (width 0.25) (layer B.Cu) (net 4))
 (segment (start 182.499 99.06) (end 183.896 100.457) (width 0.25) (layer B.Cu) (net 4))
 (segment (start 191.54 90.17) (end 191.77 90.17) (width 0.25) (layer F.Cu) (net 4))
 (segment (start 191.77 90.17) (end 192.405 90.805) (width 0.25) (layer F.Cu) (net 4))
 (segment (start 192.405 90.805) (end 192.405 94.615) (width 0.25) (layer F.Cu) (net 4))
 (segment (start 191.455 95.715) (end 191.455 94.93) (width 0.25) (layer F.Cu) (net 4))
 (segment (start 193.355 94.93) (end 193.355 95.715) (width 0.25) (layer F.Cu) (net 4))
 (segment (start 193.04 94.615) (end 193.355 94.93) (width 0.25) (layer F.Cu) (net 4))
 (segment (start 191.77 94.615) (end 192.405 94.615) (width 0.25) (layer F.Cu) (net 4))
 (segment (start 192.405 94.615) (end 193.04 94.615) (width 0.25) (layer F.Cu) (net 4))
 (segment (start 191.455 94.93) (end 191.77 94.615) (width 0.25) (layer F.Cu) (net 4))
 (segment (start 191.54 90.17) (end 191.54 90.4) (width 0.25) (layer F.Cu) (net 4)))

